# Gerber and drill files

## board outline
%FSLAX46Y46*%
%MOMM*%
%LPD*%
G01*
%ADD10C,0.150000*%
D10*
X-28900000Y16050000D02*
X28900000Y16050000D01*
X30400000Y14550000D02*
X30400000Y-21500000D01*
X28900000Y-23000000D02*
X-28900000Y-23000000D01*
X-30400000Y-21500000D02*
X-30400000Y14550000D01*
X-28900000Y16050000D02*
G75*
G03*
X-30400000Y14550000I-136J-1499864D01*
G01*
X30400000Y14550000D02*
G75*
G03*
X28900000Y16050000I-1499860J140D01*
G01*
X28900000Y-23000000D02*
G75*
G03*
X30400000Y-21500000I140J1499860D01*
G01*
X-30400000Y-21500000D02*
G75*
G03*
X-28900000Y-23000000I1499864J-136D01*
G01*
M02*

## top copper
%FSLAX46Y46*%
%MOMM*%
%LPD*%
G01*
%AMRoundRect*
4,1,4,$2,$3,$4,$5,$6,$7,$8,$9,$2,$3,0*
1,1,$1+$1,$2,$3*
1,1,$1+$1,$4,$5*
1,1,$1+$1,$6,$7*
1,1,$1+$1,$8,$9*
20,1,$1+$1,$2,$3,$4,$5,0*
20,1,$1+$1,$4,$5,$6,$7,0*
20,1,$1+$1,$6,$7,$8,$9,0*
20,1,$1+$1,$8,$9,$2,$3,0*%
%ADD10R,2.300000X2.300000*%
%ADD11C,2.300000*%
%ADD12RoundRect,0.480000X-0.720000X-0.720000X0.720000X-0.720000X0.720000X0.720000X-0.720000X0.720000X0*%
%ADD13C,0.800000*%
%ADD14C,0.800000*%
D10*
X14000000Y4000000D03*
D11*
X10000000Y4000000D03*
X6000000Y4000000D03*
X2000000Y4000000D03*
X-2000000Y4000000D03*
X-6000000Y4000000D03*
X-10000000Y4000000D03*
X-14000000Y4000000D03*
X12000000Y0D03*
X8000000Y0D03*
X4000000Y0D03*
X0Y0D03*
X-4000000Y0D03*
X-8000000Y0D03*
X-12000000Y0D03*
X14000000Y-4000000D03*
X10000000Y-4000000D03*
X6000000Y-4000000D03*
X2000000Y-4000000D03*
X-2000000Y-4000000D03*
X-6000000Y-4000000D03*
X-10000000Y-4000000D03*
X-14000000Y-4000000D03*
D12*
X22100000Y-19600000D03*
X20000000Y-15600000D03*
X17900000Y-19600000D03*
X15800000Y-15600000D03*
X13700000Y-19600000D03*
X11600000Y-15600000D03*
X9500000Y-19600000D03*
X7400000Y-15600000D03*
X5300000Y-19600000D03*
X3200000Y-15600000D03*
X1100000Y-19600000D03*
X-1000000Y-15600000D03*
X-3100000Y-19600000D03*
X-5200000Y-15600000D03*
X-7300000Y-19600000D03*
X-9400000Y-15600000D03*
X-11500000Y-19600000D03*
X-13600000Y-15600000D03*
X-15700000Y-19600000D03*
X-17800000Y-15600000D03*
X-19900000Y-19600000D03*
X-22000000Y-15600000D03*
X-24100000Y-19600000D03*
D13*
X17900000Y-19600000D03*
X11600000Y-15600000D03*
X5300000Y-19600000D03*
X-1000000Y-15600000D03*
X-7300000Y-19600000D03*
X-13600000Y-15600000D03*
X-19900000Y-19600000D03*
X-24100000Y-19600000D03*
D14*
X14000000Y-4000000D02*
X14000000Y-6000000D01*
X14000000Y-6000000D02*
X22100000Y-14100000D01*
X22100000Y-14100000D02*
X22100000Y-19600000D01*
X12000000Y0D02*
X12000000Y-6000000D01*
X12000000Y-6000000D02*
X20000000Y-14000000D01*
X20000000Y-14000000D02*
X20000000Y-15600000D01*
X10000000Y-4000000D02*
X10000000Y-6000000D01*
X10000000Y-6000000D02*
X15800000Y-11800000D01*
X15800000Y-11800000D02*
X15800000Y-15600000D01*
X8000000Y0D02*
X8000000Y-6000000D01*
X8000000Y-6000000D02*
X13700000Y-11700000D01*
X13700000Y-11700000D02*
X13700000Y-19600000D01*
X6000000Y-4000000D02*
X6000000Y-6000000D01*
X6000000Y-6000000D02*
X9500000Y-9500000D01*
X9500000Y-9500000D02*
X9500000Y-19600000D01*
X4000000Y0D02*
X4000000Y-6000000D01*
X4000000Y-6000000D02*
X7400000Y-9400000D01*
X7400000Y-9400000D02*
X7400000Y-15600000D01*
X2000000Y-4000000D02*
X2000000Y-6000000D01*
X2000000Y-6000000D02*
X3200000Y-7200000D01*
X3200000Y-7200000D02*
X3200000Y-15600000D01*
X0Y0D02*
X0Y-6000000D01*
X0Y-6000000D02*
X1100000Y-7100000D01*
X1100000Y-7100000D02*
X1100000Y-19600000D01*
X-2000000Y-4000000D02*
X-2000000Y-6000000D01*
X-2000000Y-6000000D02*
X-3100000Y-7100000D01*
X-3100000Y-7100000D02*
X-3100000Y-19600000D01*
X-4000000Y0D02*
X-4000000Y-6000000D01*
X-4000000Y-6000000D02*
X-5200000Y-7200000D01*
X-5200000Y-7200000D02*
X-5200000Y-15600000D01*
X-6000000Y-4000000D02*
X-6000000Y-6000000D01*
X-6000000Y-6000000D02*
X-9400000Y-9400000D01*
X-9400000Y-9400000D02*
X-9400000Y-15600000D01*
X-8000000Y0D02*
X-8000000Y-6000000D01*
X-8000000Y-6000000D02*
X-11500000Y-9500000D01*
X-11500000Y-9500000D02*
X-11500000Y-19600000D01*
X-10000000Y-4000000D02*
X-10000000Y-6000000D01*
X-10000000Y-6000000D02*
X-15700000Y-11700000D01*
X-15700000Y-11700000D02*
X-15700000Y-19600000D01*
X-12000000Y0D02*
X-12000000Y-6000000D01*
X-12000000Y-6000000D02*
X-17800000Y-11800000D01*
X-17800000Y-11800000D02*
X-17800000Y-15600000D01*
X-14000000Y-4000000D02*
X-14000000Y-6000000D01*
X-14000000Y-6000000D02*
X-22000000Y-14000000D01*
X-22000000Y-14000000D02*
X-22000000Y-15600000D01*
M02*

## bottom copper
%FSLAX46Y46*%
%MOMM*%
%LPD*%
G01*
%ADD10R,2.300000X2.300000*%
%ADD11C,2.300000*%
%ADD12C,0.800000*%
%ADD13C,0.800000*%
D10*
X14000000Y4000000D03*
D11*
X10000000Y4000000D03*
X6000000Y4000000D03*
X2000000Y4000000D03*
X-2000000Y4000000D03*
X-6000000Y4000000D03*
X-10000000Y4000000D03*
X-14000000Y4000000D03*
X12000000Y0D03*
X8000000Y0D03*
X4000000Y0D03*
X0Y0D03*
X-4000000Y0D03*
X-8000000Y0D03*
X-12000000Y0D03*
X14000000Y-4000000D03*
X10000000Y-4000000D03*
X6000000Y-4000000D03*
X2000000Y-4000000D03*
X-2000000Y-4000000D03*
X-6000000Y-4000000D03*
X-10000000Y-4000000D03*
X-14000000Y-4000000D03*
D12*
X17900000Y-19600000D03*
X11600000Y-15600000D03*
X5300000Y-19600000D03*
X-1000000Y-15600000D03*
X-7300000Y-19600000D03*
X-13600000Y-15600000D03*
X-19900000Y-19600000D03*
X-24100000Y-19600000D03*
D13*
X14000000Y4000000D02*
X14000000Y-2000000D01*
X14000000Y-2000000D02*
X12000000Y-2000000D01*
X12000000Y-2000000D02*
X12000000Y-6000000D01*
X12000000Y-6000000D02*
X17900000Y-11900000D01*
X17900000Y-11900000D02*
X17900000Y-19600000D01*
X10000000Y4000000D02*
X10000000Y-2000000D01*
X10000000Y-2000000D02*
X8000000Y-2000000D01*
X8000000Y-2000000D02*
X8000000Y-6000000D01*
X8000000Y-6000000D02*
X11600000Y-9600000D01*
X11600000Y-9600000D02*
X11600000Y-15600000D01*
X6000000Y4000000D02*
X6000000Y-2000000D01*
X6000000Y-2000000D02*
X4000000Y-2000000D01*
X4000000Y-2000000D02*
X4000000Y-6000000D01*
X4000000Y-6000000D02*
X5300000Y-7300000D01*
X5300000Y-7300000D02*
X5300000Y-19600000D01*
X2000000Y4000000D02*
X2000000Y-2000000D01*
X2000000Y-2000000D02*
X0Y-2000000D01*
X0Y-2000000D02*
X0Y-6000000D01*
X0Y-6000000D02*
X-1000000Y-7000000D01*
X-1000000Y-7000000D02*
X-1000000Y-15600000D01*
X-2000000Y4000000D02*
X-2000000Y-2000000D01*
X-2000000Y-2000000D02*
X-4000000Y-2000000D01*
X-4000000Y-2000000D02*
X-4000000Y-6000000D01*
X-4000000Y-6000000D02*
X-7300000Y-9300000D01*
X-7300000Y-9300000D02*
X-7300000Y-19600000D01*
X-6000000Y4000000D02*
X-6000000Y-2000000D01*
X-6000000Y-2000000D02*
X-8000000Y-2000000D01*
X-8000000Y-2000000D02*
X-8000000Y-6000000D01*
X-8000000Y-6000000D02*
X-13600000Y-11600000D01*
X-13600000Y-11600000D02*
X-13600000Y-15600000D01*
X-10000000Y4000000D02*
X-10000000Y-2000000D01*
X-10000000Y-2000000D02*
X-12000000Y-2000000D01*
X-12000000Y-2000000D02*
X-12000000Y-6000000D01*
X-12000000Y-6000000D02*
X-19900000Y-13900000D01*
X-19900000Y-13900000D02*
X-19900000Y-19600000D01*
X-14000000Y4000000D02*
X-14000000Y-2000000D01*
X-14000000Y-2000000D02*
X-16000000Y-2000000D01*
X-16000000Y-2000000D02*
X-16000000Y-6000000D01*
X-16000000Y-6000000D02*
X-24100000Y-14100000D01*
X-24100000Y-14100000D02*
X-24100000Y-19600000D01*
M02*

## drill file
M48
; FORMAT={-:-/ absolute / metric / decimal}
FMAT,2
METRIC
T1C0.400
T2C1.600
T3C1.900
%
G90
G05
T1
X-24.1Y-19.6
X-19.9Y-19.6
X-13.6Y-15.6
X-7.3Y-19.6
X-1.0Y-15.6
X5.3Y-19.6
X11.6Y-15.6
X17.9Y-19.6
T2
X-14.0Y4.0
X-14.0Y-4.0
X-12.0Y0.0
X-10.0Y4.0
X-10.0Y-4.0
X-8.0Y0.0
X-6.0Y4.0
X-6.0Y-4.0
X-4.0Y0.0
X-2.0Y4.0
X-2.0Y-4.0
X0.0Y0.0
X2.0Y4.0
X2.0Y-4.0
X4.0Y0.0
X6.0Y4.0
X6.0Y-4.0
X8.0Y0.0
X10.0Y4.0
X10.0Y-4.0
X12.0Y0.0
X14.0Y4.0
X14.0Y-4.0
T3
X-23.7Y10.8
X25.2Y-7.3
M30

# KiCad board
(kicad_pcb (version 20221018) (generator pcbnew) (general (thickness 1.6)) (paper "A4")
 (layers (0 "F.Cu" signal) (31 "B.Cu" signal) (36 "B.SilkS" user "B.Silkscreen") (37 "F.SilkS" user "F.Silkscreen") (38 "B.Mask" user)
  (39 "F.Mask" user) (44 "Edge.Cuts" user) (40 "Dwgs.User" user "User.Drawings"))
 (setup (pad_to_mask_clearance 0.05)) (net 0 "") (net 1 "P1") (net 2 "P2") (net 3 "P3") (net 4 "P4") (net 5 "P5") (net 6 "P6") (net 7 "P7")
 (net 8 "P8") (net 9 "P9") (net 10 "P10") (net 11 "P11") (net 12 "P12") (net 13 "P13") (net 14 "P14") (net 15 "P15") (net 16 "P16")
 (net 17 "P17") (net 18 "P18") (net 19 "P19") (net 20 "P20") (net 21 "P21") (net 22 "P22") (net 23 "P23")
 (gr_line (start -28.9 -16.05) (end 28.9 -16.05) (layer "Edge.Cuts") (width 0.15))
 (gr_line (start 30.4 -14.55) (end 30.4 21.5) (layer "Edge.Cuts") (width 0.15))
 (gr_line (start 28.9 23.0) (end -28.9 23.0) (layer "Edge.Cuts") (width 0.15))
 (gr_line (start -30.4 21.5) (end -30.4 -14.55) (layer "Edge.Cuts") (width 0.15))
 (gr_arc (start -30.4000 -14.5500) (mid -29.9607 -15.6107) (end -28.9000 -16.0500) (layer "Edge.Cuts") (width 0.15))
 (gr_arc (start 30.4000 -14.5500) (mid 29.9607 -15.6107) (end 28.9000 -16.0500) (layer "Edge.Cuts") (width 0.15))
 (gr_arc (start 30.4000 21.5000) (mid 29.9607 22.5607) (end 28.9000 23.0000) (layer "Edge.Cuts") (width 0.15))
 (gr_arc (start -30.4000 21.5000) (mid -29.9607 22.5607) (end -28.9000 23.0000) (layer "Edge.Cuts") (width 0.15))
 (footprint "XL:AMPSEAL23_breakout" (layer "F.Cu") (at 0 0)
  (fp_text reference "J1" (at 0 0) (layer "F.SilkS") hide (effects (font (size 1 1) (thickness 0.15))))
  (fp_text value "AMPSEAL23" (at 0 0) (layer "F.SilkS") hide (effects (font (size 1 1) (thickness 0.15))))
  (pad "1" thru_hole rect (at 14 -4.0) (size 2.3 2.3) (drill 1.6) (layers "*.Cu" "*.Mask") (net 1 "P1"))
  (pad "2" thru_hole circle (at 10 -4.0) (size 2.3 2.3) (drill 1.6) (layers "*.Cu" "*.Mask") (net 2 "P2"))
  (pad "3" thru_hole circle (at 6 -4.0) (size 2.3 2.3) (drill 1.6) (layers "*.Cu" "*.Mask") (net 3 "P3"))
  (pad "4" thru_hole circle (at 2 -4.0) (size 2.3 2.3) (drill 1.6) (layers "*.Cu" "*.Mask") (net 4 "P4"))
  (pad "5" thru_hole circle (at -2 -4.0) (size 2.3 2.3) (drill 1.6) (layers "*.Cu" "*.Mask") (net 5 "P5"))
  (pad "6" thru_hole circle (at -6 -4.0) (size 2.3 2.3) (drill 1.6) (layers "*.Cu" "*.Mask") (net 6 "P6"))
  (pad "7" thru_hole circle (at -10 -4.0) (size 2.3 2.3) (drill 1.6) (layers "*.Cu" "*.Mask") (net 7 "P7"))
  (pad "8" thru_hole circle (at -14 -4.0) (size 2.3 2.3) (drill 1.6) (layers "*.Cu" "*.Mask") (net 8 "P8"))
  (pad "9" thru_hole circle (at 12 -0.0) (size 2.3 2.3) (drill 1.6) (layers "*.Cu" "*.Mask") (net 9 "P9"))
  (pad "10" thru_hole circle (at 8 -0.0) (size 2.3 2.3) (drill 1.6) (layers "*.Cu" "*.Mask") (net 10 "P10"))
  (pad "11" thru_hole circle (at 4 -0.0) (size 2.3 2.3) (drill 1.6) (layers "*.Cu" "*.Mask") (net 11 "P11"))
  (pad "12" thru_hole circle (at 0 -0.0) (size 2.3 2.3) (drill 1.6) (layers "*.Cu" "*.Mask") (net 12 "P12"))
  (pad "13" thru_hole circle (at -4 -0.0) (size 2.3 2.3) (drill 1.6) (layers "*.Cu" "*.Mask") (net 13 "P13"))
  (pad "14" thru_hole circle (at -8 -0.0) (size 2.3 2.3) (drill 1.6) (layers "*.Cu" "*.Mask") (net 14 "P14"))
  (pad "15" thru_hole circle (at -12 -0.0) (size 2.3 2.3) (drill 1.6) (layers "*.Cu" "*.Mask") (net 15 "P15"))
  (pad "16" thru_hole circle (at 14 4.0) (size 2.3 2.3) (drill 1.6) (layers "*.Cu" "*.Mask") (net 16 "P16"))
  (pad "17" thru_hole circle (at 10 4.0) (size 2.3 2.3) (drill 1.6) (layers "*.Cu" "*.Mask") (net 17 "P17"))
  (pad "18" thru_hole circle (at 6 4.0) (size 2.3 2.3) (drill 1.6) (layers "*.Cu" "*.Mask") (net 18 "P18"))
  (pad "19" thru_hole circle (at 2 4.0) (size 2.3 2.3) (drill 1.6) (layers "*.Cu" "*.Mask") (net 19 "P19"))
  (pad "20" thru_hole circle (at -2 4.0) (size 2.3 2.3) (drill 1.6) (layers "*.Cu" "*.Mask") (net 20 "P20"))
  (pad "21" thru_hole circle (at -6 4.0) (size 2.3 2.3) (drill 1.6) (layers "*.Cu" "*.Mask") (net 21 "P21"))
  (pad "22" thru_hole circle (at -10 4.0) (size 2.3 2.3) (drill 1.6) (layers "*.Cu" "*.Mask") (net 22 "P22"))
  (pad "23" thru_hole circle (at -14 4.0) (size 2.3 2.3) (drill 1.6) (layers "*.Cu" "*.Mask") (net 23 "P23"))
  (pad "" np_thru_hole circle (at -23.7 -10.8) (size 1.9 1.9) (drill 1.9) (layers "*.Cu" "*.Mask"))
  (pad "" np_thru_hole circle (at 25.2 7.3) (size 1.9 1.9) (drill 1.9) (layers "*.Cu" "*.Mask"))
  (pad "16" smd roundrect (at 22.1 19.6) (size 2.4 2.4) (layers "F.Cu" "F.Mask") (roundrect_rratio 0.2) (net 16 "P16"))
  (pad "9" smd roundrect (at 20.0 15.6) (size 2.4 2.4) (layers "F.Cu" "F.Mask") (roundrect_rratio 0.2) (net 9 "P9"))
  (pad "1" smd roundrect (at 17.9 19.6) (size 2.4 2.4) (layers "F.Cu" "F.Mask") (roundrect_rratio 0.2) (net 1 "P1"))
  (pad "17" smd roundrect (at 15.8 15.6) (size 2.4 2.4) (layers "F.Cu" "F.Mask") (roundrect_rratio 0.2) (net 17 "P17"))
  (pad "10" smd roundrect (at 13.7 19.6) (size 2.4 2.4) (layers "F.Cu" "F.Mask") (roundrect_rratio 0.2) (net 10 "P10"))
  (pad "2" smd roundrect (at 11.6 15.6) (size 2.4 2.4) (layers "F.Cu" "F.Mask") (roundrect_rratio 0.2) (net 2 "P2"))
  (pad "18" smd roundrect (at 9.5 19.6) (size 2.4 2.4) (layers "F.Cu" "F.Mask") (roundrect_rratio 0.2) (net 18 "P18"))
  (pad "11" smd roundrect (at 7.4 15.6) (size 2.4 2.4) (layers "F.Cu" "F.Mask") (roundrect_rratio 0.2) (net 11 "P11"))
  (pad "3" smd roundrect (at 5.3 19.6) (size 2.4 2.4) (layers "F.Cu" "F.Mask") (roundrect_rratio 0.2) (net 3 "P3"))
  (pad "19" smd roundrect (at 3.2 15.6) (size 2.4 2.4) (layers "F.Cu" "F.Mask") (roundrect_rratio 0.2) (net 19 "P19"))
  (pad "12" smd roundrect (at 1.1 19.6) (size 2.4 2.4) (layers "F.Cu" "F.Mask") (roundrect_rratio 0.2) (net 12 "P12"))
  (pad "4" smd roundrect (at -1.0 15.6) (size 2.4 2.4) (layers "F.Cu" "F.Mask") (roundrect_rratio 0.2) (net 4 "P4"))
  (pad "20" smd roundrect (at -3.1 19.6) (size 2.4 2.4) (layers "F.Cu" "F.Mask") (roundrect_rratio 0.2) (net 20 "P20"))
  (pad "13" smd roundrect (at -5.2 15.6) (size 2.4 2.4) (layers "F.Cu" "F.Mask") (roundrect_rratio 0.2) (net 13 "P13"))
  (pad "5" smd roundrect (at -7.3 19.6) (size 2.4 2.4) (layers "F.Cu" "F.Mask") (roundrect_rratio 0.2) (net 5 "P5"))
  (pad "21" smd roundrect (at -9.4 15.6) (size 2.4 2.4) (layers "F.Cu" "F.Mask") (roundrect_rratio 0.2) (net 21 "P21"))
  (pad "14" smd roundrect (at -11.5 19.6) (size 2.4 2.4) (layers "F.Cu" "F.Mask") (roundrect_rratio 0.2) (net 14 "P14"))
  (pad "6" smd roundrect (at -13.6 15.6) (size 2.4 2.4) (layers "F.Cu" "F.Mask") (roundrect_rratio 0.2) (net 6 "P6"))
  (pad "22" smd roundrect (at -15.7 19.6) (size 2.4 2.4) (layers "F.Cu" "F.Mask") (roundrect_rratio 0.2) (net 22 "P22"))
  (pad "15" smd roundrect (at -17.8 15.6) (size 2.4 2.4) (layers "F.Cu" "F.Mask") (roundrect_rratio 0.2) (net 15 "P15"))
  (pad "7" smd roundrect (at -19.9 19.6) (size 2.4 2.4) (layers "F.Cu" "F.Mask") (roundrect_rratio 0.2) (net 7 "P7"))
  (pad "23" smd roundrect (at -22.0 15.6) (size 2.4 2.4) (layers "F.Cu" "F.Mask") (roundrect_rratio 0.2) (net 23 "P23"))
  (pad "8" smd roundrect (at -24.1 19.6) (size 2.4 2.4) (layers "F.Cu" "F.Mask") (roundrect_rratio 0.2) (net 8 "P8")))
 (segment (start 14 4.0) (end 14.0 6.0) (width 0.8) (layer "F.Cu") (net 16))
 (segment (start 14.0 6.0) (end 22.1 14.1) (width 0.8) (layer "F.Cu") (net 16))
 (segment (start 22.1 14.1) (end 22.1 19.6) (width 0.8) (layer "F.Cu") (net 16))
 (segment (start 12 -0.0) (end 12.0 6.0) (width 0.8) (layer "F.Cu") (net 9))
 (segment (start 12.0 6.0) (end 20.0 14.0) (width 0.8) (layer "F.Cu") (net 9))
 (segment (start 20.0 14.0) (end 20.0 15.6) (width 0.8) (layer "F.Cu") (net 9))
 (segment (start 14 -4.0) (end 14 2.0) (width 0.8) (layer "B.Cu") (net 1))
 (segment (start 14 2.0) (end 12.0 2.0) (width 0.8) (layer "B.Cu") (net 1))
 (segment (start 12.0 2.0) (end 12.0 6.0) (width 0.8) (layer "B.Cu") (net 1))
 (segment (start 12.0 6.0) (end 17.9 11.9) (width 0.8) (layer "B.Cu") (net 1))
 (segment (start 17.9 11.9) (end 17.9 19.6) (width 0.8) (layer "B.Cu") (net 1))
 (via (at 17.9 19.6) (size 0.8) (drill 0.4) (layers "F.Cu" "B.Cu") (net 1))
 (segment (start 10 4.0) (end 10.0 6.0) (width 0.8) (layer "F.Cu") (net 17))
 (segment (start 10.0 6.0) (end 15.8 11.8) (width 0.8) (layer "F.Cu") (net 17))
 (segment (start 15.8 11.8) (end 15.8 15.6) (width 0.8) (layer "F.Cu") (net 17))
 (segment (start 8 -0.0) (end 8.0 6.0) (width 0.8) (layer "F.Cu") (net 10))
 (segment (start 8.0 6.0) (end 13.7 11.7) (width 0.8) (layer "F.Cu") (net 10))
 (segment (start 13.7 11.7) (end 13.7 19.6) (width 0.8) (layer "F.Cu") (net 10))
 (segment (start 10 -4.0) (end 10 2.0) (width 0.8) (layer "B.Cu") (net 2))
 (segment (start 10 2.0) (end 8.0 2.0) (width 0.8) (layer "B.Cu") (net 2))
 (segment (start 8.0 2.0) (end 8.0 6.0) (width 0.8) (layer "B.Cu") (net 2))
 (segment (start 8.0 6.0) (end 11.6 9.6) (width 0.8) (layer "B.Cu") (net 2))
 (segment (start 11.6 9.6) (end 11.6 15.6) (width 0.8) (layer "B.Cu") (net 2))
 (via (at 11.6 15.6) (size 0.8) (drill 0.4) (layers "F.Cu" "B.Cu") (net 2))
 (segment (start 6 4.0) (end 6.0 6.0) (width 0.8) (layer "F.Cu") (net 18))
 (segment (start 6.0 6.0) (end 9.5 9.5) (width 0.8) (layer "F.Cu") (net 18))
 (segment (start 9.5 9.5) (end 9.5 19.6) (width 0.8) (layer "F.Cu") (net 18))
 (segment (start 4 -0.0) (end 4.0 6.0) (width 0.8) (layer "F.Cu") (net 11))
 (segment (start 4.0 6.0) (end 7.4 9.4) (width 0.8) (layer "F.Cu") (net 11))
 (segment (start 7.4 9.4) (end 7.4 15.6) (width 0.8) (layer "F.Cu") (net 11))
 (segment (start 6 -4.0) (end 6 2.0) (width 0.8) (layer "B.Cu") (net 3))
 (segment (start 6 2.0) (end 4.0 2.0) (width 0.8) (layer "B.Cu") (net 3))
 (segment (start 4.0 2.0) (end 4.0 6.0) (width 0.8) (layer "B.Cu") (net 3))
 (segment (start 4.0 6.0) (end 5.3 7.3) (width 0.8) (layer "B.Cu") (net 3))
 (segment (start 5.3 7.3) (end 5.3 19.6) (width 0.8) (layer "B.Cu") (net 3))
 (via (at 5.3 19.6) (size 0.8) (drill 0.4) (layers "F.Cu" "B.Cu") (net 3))
 (segment (start 2 4.0) (end 2.0 6.0) (width 0.8) (layer "F.Cu") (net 19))
 (segment (start 2.0 6.0) (end 3.2 7.2) (width 0.8) (layer "F.Cu") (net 19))
 (segment (start 3.2 7.2) (end 3.2 15.6) (width 0.8) (layer "F.Cu") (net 19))
 (segment (start 0 -0.0) (end -0.0 6.0) (width 0.8) (layer "F.Cu") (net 12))
 (segment (start -0.0 6.0) (end 1.1 7.1) (width 0.8) (layer "F.Cu") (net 12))
 (segment (start 1.1 7.1) (end 1.1 19.6) (width 0.8) (layer "F.Cu") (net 12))
 (segment (start 2 -4.0) (end 2 2.0) (width 0.8) (layer "B.Cu") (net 4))
 (segment (start 2 2.0) (end -0.0 2.0) (width 0.8) (layer "B.Cu") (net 4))
 (segment (start -0.0 2.0) (end -0.0 6.0) (width 0.8) (layer "B.Cu") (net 4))
 (segment (start -0.0 6.0) (end -1.0 7.0) (width 0.8) (layer "B.Cu") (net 4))
 (segment (start -1.0 7.0) (end -1.0 15.6) (width 0.8) (layer "B.Cu") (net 4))
 (via (at -1.0 15.6) (size 0.8) (drill 0.4) (layers "F.Cu" "B.Cu") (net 4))
 (segment (start -2 4.0) (end -2.0 6.0) (width 0.8) (layer "F.Cu") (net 20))
 (segment (start -2.0 6.0) (end -3.1 7.1) (width 0.8) (layer "F.Cu") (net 20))
 (segment (start -3.1 7.1) (end -3.1 19.6) (width 0.8) (layer "F.Cu") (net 20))
 (segment (start -4 -0.0) (end -4.0 6.0) (width 0.8) (layer "F.Cu") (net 13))
 (segment (start -4.0 6.0) (end -5.2 7.2) (width 0.8) (layer "F.Cu") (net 13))
 (segment (start -5.2 7.2) (end -5.2 15.6) (width 0.8) (layer "F.Cu") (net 13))
 (segment (start -2 -4.0) (end -2 2.0) (width 0.8) (layer "B.Cu") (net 5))
 (segment (start -2 2.0) (end -4.0 2.0) (width 0.8) (layer "B.Cu") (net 5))
 (segment (start -4.0 2.0) (end -4.0 6.0) (width 0.8) (layer "B.Cu") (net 5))
 (segment (start -4.0 6.0) (end -7.3 9.3) (width 0.8) (layer "B.Cu") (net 5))
 (segment (start -7.3 9.3) (end -7.3 19.6) (width 0.8) (layer "B.Cu") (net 5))
 (via (at -7.3 19.6) (size 0.8) (drill 0.4) (layers "F.Cu" "B.Cu") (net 5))
 (segment (start -6 4.0) (end -6.0 6.0) (width 0.8) (layer "F.Cu") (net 21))
 (segment (start -6.0 6.0) (end -9.4 9.4) (width 0.8) (layer "F.Cu") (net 21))
 (segment (start -9.4 9.4) (end -9.4 15.6) (width 0.8) (layer "F.Cu") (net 21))
 (segment (start -8 -0.0) (end -8.0 6.0) (width 0.8) (layer "F.Cu") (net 14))
 (segment (start -8.0 6.0) (end -11.5 9.5) (width 0.8) (layer "F.Cu") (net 14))
 (segment (start -11.5 9.5) (end -11.5 19.6) (width 0.8) (layer "F.Cu") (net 14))
 (segment (start -6 -4.0) (end -6 2.0) (width 0.8) (layer "B.Cu") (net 6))
 (segment (start -6 2.0) (end -8.0 2.0) (width 0.8) (layer "B.Cu") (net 6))
 (segment (start -8.0 2.0) (end -8.0 6.0) (width 0.8) (layer "B.Cu") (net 6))
 (segment (start -8.0 6.0) (end -13.6 11.6) (width 0.8) (layer "B.Cu") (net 6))
 (segment (start -13.6 11.6) (end -13.6 15.6) (width 0.8) (layer "B.Cu") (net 6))
 (via (at -13.6 15.6) (size 0.8) (drill 0.4) (layers "F.Cu" "B.Cu") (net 6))
 (segment (start -10 4.0) (end -10.0 6.0) (width 0.8) (layer "F.Cu") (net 22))
 (segment (start -10.0 6.0) (end -15.7 11.7) (width 0.8) (layer "F.Cu") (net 22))
 (segment (start -15.7 11.7) (end -15.7 19.6) (width 0.8) (layer "F.Cu") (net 22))
 (segment (start -12 -0.0) (end -12.0 6.0) (width 0.8) (layer "F.Cu") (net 15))
 (segment (start -12.0 6.0) (end -17.8 11.8) (width 0.8) (layer "F.Cu") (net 15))
 (segment (start -17.8 11.8) (end -17.8 15.6) (width 0.8) (layer "F.Cu") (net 15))
 (segment (start -10 -4.0) (end -10 2.0) (width 0.8) (layer "B.Cu") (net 7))
 (segment (start -10 2.0) (end -12.0 2.0) (width 0.8) (layer "B.Cu") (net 7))
 (segment (start -12.0 2.0) (end -12.0 6.0) (width 0.8) (layer "B.Cu") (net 7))
 (segment (start -12.0 6.0) (end -19.9 13.9) (width 0.8) (layer "B.Cu") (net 7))
 (segment (start -19.9 13.9) (end -19.9 19.6) (width 0.8) (layer "B.Cu") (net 7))
 (via (at -19.9 19.6) (size 0.8) (drill 0.4) (layers "F.Cu" "B.Cu") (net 7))
 (segment (start -14 4.0) (end -14.0 6.0) (width 0.8) (layer "F.Cu") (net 23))
 (segment (start -14.0 6.0) (end -22.0 14.0) (width 0.8) (layer "F.Cu") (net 23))
 (segment (start -22.0 14.0) (end -22.0 15.6) (width 0.8) (layer "F.Cu") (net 23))
 (segment (start -14 -4.0) (end -14 2.0) (width 0.8) (layer "B.Cu") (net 8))
 (segment (start -14 2.0) (end -16.0 2.0) (width 0.8) (layer "B.Cu") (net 8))
 (segment (start -16.0 2.0) (end -16.0 6.0) (width 0.8) (layer "B.Cu") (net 8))
 (segment (start -16.0 6.0) (end -24.1 14.1) (width 0.8) (layer "B.Cu") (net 8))
 (segment (start -24.1 14.1) (end -24.1 19.6) (width 0.8) (layer "B.Cu") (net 8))
 (via (at -24.1 19.6) (size 0.8) (drill 0.4) (layers "F.Cu" "B.Cu") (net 8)))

